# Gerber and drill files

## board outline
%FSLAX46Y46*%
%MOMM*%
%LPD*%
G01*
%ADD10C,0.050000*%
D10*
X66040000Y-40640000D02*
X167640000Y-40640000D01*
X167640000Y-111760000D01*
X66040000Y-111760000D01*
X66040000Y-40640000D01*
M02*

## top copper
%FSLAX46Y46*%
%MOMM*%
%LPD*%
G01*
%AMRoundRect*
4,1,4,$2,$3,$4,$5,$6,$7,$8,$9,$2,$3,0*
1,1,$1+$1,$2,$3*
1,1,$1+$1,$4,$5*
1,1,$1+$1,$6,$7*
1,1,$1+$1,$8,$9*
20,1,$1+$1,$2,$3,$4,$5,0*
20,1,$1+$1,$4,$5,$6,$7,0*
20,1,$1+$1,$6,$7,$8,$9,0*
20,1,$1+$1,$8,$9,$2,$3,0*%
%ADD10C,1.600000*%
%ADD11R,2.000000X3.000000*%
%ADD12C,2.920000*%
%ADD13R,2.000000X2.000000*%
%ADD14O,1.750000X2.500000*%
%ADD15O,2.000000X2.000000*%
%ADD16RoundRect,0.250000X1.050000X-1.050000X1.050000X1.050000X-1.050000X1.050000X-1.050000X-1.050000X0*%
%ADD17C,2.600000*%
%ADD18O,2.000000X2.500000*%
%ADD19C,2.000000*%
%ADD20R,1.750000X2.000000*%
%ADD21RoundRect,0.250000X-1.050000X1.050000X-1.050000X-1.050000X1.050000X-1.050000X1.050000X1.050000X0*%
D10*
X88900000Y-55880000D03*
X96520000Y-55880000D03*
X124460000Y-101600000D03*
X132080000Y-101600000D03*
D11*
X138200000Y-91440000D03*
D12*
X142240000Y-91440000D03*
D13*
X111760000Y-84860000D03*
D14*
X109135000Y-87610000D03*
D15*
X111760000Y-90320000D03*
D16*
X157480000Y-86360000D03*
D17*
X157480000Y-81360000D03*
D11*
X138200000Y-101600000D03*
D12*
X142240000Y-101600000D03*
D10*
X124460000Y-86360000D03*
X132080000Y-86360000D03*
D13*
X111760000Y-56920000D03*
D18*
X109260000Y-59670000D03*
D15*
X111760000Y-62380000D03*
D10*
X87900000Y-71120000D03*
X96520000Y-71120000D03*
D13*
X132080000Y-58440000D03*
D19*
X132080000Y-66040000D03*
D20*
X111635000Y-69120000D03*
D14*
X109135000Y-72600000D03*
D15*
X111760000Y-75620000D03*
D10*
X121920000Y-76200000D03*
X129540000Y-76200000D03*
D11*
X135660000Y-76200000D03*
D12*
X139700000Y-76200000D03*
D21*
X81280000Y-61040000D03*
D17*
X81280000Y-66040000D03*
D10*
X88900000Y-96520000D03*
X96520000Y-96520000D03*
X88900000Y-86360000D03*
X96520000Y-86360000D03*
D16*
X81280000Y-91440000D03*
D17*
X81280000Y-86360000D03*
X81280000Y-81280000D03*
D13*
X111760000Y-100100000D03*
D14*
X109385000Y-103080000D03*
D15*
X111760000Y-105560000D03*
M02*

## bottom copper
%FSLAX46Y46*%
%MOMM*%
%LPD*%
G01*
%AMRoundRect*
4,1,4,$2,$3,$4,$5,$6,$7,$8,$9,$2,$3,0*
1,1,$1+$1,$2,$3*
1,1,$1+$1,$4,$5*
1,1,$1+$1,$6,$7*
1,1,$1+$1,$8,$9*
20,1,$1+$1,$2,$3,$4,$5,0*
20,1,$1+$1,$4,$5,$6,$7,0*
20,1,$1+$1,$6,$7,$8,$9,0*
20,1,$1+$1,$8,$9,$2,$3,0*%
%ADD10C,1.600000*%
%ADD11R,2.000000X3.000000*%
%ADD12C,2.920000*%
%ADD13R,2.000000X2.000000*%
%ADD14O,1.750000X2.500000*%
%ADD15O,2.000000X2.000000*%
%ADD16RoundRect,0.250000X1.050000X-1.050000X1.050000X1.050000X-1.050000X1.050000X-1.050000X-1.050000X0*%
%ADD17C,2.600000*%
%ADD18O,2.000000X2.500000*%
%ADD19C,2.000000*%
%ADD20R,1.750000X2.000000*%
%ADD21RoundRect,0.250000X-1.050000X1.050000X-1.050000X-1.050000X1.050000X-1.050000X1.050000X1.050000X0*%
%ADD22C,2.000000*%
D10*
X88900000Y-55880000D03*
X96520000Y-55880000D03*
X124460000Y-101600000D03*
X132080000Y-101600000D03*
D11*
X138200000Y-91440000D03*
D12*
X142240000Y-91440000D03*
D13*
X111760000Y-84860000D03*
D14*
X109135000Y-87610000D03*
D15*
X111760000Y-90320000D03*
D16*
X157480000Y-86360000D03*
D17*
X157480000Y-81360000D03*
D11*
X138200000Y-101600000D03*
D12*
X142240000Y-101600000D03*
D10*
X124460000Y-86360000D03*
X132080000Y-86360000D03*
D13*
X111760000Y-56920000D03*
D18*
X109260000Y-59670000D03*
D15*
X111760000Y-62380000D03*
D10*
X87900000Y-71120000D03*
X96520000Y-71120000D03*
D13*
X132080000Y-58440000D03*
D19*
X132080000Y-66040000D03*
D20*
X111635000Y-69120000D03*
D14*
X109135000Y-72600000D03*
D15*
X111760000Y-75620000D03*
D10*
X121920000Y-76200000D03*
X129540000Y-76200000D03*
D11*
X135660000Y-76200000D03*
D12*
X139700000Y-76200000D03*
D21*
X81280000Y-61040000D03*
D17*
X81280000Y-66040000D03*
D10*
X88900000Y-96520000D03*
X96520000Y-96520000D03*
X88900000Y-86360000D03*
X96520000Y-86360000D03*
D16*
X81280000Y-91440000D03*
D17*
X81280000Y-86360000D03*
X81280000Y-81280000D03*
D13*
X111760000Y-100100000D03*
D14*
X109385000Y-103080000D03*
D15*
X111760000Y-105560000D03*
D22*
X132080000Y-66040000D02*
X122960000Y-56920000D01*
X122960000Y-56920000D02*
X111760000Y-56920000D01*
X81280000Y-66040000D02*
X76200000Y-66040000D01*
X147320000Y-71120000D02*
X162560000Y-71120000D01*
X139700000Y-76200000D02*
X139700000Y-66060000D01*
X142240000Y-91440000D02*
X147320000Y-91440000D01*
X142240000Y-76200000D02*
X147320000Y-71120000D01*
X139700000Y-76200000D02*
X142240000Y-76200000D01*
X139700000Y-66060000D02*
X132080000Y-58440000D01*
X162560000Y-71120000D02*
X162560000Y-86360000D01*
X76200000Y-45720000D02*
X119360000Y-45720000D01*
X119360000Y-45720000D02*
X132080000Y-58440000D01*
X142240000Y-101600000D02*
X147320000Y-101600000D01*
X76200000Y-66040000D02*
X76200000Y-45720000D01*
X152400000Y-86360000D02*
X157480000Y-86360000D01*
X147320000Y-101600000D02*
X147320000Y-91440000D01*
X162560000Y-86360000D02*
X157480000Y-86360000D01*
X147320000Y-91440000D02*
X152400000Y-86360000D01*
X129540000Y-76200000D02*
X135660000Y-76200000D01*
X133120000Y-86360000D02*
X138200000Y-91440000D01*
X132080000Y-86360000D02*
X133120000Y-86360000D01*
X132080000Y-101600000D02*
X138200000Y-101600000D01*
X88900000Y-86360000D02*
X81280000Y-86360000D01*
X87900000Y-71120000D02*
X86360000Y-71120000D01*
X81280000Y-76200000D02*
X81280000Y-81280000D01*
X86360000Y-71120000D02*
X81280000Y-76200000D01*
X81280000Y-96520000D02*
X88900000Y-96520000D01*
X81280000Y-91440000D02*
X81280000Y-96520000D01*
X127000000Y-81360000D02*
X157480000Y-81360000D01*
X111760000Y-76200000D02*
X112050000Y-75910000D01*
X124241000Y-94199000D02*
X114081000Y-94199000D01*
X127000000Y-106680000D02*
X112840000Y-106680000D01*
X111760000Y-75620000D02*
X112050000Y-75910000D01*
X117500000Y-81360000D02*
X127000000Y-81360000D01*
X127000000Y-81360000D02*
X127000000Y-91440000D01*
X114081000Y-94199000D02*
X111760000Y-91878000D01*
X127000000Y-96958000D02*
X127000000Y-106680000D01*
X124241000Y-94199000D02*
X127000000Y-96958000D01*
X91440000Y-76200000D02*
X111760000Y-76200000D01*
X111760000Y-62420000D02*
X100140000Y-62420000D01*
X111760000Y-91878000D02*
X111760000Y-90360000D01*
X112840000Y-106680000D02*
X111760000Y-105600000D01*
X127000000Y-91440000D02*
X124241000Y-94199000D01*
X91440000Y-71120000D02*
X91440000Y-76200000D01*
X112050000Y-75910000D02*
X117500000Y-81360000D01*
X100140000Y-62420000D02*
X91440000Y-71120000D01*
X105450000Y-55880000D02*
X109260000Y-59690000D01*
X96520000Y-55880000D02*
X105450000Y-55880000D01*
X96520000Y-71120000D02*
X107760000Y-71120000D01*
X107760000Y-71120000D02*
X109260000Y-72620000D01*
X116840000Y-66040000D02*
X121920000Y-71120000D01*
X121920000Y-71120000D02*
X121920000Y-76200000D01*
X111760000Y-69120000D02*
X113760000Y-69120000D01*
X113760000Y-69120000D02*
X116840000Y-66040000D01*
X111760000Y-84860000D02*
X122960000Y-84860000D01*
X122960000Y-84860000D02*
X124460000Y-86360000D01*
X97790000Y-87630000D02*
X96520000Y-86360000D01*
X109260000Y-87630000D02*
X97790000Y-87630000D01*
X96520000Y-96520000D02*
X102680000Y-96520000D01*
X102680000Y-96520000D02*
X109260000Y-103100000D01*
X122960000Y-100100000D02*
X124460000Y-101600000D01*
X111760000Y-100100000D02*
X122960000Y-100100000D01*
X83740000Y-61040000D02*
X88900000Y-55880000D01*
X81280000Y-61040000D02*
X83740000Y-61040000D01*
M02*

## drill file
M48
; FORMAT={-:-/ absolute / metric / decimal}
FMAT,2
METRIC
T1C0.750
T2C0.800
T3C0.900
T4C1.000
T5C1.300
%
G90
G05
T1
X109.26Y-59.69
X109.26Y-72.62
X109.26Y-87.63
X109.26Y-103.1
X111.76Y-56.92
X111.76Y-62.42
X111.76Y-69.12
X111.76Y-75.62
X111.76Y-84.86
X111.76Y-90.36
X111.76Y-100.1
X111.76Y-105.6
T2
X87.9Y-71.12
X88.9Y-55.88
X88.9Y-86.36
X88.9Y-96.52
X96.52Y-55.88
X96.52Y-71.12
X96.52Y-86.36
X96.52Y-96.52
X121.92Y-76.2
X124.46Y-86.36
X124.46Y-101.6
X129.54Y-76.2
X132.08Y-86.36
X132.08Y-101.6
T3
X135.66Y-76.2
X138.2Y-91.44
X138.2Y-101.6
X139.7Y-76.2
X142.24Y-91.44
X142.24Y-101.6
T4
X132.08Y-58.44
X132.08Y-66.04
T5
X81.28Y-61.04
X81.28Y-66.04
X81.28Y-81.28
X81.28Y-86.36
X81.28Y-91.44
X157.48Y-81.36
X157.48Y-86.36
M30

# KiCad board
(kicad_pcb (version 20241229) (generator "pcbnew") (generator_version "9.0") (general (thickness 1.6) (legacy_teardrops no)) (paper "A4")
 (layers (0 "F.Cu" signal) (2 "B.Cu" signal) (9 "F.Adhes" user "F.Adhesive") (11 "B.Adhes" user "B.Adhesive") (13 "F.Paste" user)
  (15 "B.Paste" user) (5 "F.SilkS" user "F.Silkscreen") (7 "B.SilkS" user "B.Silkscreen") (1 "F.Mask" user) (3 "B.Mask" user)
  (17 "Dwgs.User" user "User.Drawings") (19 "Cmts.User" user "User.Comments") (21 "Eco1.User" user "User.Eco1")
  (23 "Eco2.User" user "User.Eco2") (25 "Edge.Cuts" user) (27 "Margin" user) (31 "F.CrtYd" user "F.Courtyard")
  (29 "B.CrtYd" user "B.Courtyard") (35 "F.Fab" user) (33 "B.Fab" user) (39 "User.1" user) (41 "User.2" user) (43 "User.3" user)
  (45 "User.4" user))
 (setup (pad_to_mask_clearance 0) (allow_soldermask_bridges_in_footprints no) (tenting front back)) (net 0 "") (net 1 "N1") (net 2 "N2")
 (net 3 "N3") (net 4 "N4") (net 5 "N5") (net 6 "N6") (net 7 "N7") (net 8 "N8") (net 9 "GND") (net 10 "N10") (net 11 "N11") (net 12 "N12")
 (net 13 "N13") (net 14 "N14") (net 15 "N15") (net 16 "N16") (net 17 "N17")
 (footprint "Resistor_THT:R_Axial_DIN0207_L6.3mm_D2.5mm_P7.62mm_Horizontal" (layer "F.Cu") (at 88.9 55.88)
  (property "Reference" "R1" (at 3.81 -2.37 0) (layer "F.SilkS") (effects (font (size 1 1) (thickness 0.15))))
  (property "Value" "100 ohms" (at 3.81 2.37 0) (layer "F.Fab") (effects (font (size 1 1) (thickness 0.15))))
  (pad "1" thru_hole circle (at 0 0) (size 1.6 1.6) (drill 0.8) (layers "*.Cu" "*.Mask") (remove_unused_layers no) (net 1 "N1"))
  (pad "2" thru_hole circle (at 7.62 0) (size 1.6 1.6) (drill 0.8) (layers "*.Cu" "*.Mask") (remove_unused_layers no) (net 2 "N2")))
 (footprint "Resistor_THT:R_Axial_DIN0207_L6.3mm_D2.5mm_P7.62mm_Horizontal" (layer "F.Cu") (at 124.46 101.6)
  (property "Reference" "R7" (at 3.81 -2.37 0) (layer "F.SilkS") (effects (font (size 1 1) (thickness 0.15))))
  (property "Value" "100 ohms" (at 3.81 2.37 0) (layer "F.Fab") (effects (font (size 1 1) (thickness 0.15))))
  (pad "1" thru_hole circle (at 0 0) (size 1.6 1.6) (drill 0.8) (layers "*.Cu" "*.Mask") (remove_unused_layers no) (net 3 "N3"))
  (pad "2" thru_hole circle (at 7.62 0) (size 1.6 1.6) (drill 0.8) (layers "*.Cu" "*.Mask") (remove_unused_layers no) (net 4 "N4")))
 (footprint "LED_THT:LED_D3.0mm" (layer "F.Cu") (at 139.7 91.44)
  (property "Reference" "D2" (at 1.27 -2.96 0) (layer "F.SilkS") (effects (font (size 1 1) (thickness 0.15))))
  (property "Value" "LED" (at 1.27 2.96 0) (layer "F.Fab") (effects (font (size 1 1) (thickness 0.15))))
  (pad "1" thru_hole rect (at -1.5 0) (size 2 3) (drill 0.9) (layers "*.Cu" "*.Mask") (remove_unused_layers no) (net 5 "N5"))
  (pad "2" thru_hole circle (at 2.54 0) (size 2.92 2.92) (drill 0.9) (layers "*.Cu" "*.Mask") (remove_unused_layers no) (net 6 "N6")))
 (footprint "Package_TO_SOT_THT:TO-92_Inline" (layer "F.Cu") (at 111.76 86.36 -90)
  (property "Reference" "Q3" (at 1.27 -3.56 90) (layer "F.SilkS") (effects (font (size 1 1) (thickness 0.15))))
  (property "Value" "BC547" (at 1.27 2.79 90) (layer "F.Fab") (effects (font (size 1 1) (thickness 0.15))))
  (pad "1" thru_hole rect (at -1.5 0 270) (size 2 2) (drill 0.75) (layers "*.Cu" "*.Mask") (remove_unused_layers no) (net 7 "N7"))
  (pad "2" thru_hole oval (at 1.27 2.5 270) (size 2.5 1.75) (drill 0.75 (offset -0.02 0.125)) (layers "*.Cu" "*.Mask")
   (remove_unused_layers no) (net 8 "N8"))
  (pad "3" thru_hole oval (at 4 0 270) (size 2 2) (drill 0.75 (offset -0.04 0)) (layers "*.Cu" "*.Mask") (remove_unused_layers no)
   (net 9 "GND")))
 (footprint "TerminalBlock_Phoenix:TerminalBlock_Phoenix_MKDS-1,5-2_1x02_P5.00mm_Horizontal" (layer "F.Cu") (at 157.48 86.36 90)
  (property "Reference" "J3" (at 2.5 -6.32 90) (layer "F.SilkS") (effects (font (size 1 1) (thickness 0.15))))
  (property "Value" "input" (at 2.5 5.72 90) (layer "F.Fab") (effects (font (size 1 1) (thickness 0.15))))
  (pad "1" thru_hole roundrect (at 0 0 90) (size 2.6 2.6) (drill 1.3) (layers "*.Cu" "*.Mask") (remove_unused_layers no)
   (roundrect_rratio 0.096154) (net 6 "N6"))
  (pad "2" thru_hole circle (at 5 0 90) (size 2.6 2.6) (drill 1.3) (layers "*.Cu" "*.Mask") (remove_unused_layers no) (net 9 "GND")))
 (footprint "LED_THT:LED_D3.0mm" (layer "F.Cu") (at 139.7 101.6)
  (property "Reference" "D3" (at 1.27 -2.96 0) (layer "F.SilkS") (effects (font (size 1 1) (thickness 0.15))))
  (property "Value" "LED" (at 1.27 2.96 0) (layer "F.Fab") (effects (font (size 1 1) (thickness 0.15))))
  (pad "1" thru_hole rect (at -1.5 0) (size 2 3) (drill 0.9) (layers "*.Cu" "*.Mask") (remove_unused_layers no) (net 4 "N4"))
  (pad "2" thru_hole circle (at 2.54 0) (size 2.92 2.92) (drill 0.9) (layers "*.Cu" "*.Mask") (remove_unused_layers no) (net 6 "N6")))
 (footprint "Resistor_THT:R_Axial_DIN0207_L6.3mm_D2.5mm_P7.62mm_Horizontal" (layer "F.Cu") (at 124.46 86.36)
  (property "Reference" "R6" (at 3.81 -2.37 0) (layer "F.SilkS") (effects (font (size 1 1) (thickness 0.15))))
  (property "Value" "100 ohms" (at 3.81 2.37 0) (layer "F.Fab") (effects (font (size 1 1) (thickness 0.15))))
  (pad "1" thru_hole circle (at 0 0) (size 1.6 1.6) (drill 0.8) (layers "*.Cu" "*.Mask") (remove_unused_layers no) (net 7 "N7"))
  (pad "2" thru_hole circle (at 7.62 0) (size 1.6 1.6) (drill 0.8) (layers "*.Cu" "*.Mask") (remove_unused_layers no) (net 5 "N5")))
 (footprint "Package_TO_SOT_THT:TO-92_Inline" (layer "F.Cu") (at 111.76 58.42 -90)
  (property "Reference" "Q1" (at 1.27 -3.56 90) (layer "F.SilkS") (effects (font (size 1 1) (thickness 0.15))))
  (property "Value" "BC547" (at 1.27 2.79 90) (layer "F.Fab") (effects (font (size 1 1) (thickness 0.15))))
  (pad "1" thru_hole rect (at -1.5 0 270) (size 2 2) (drill 0.75) (layers "*.Cu" "*.Mask") (remove_unused_layers no) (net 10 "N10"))
  (pad "2" thru_hole oval (at 1.27 2.5 270) (size 2.5 2) (drill 0.75 (offset -0.02 0)) (layers "*.Cu" "*.Mask") (remove_unused_layers no)
   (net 2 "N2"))
  (pad "3" thru_hole oval (at 4 0 270) (size 2 2) (drill 0.75 (offset -0.04 0)) (layers "*.Cu" "*.Mask") (remove_unused_layers no)
   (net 9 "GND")))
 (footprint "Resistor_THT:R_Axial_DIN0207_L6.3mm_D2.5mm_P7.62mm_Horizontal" (layer "F.Cu") (at 88.9 71.12)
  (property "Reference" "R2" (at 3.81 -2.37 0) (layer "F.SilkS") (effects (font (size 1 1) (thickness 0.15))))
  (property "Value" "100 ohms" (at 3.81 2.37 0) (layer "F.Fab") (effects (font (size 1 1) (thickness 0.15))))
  (pad "1" thru_hole circle (at -1 0) (size 1.6 1.6) (drill 0.8) (layers "*.Cu" "*.Mask") (remove_unused_layers no) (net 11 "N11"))
  (pad "2" thru_hole circle (at 7.62 0) (size 1.6 1.6) (drill 0.8) (layers "*.Cu" "*.Mask") (remove_unused_layers no) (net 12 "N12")))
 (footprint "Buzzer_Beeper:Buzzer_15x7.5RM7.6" (layer "F.Cu") (at 132.08 58.44 -90)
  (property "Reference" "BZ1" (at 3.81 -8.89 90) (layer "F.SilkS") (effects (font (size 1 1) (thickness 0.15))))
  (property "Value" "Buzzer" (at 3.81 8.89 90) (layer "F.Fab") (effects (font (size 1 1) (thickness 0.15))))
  (pad "1" thru_hole rect (at 0 0 270) (size 2 2) (drill 1) (layers "*.Cu" "*.Mask") (remove_unused_layers no) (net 6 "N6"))
  (pad "2" thru_hole circle (at 7.6 0 270) (size 2 2) (drill 1) (layers "*.Cu" "*.Mask") (remove_unused_layers no) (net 10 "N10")))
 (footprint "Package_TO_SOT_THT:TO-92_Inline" (layer "F.Cu") (at 111.76 71.12 -90)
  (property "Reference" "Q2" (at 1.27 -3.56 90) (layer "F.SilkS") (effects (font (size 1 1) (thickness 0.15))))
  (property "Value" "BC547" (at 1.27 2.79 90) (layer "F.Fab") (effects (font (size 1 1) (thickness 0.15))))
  (pad "1" thru_hole rect (at -2 0 270) (size 2 1.75) (drill 0.75 (offset 0 0.125)) (layers "*.Cu" "*.Mask") (remove_unused_layers no)
   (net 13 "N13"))
  (pad "2" thru_hole oval (at 1.5 2.5 270) (size 2.5 1.75) (drill 0.75 (offset -0.02 0.125)) (layers "*.Cu" "*.Mask")
   (remove_unused_layers no) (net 12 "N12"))
  (pad "3" thru_hole oval (at 4.5 0 270) (size 2 2) (drill 0.75) (layers "*.Cu" "*.Mask") (remove_unused_layers no) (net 9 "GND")))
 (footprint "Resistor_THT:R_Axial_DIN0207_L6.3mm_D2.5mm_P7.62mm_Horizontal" (layer "F.Cu") (at 121.92 76.2)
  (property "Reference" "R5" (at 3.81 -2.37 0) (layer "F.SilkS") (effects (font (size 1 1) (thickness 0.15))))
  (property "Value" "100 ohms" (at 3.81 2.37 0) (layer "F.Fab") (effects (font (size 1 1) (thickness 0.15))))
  (pad "1" thru_hole circle (at 0 0) (size 1.6 1.6) (drill 0.8) (layers "*.Cu" "*.Mask") (remove_unused_layers no) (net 13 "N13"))
  (pad "2" thru_hole circle (at 7.62 0) (size 1.6 1.6) (drill 0.8) (layers "*.Cu" "*.Mask") (remove_unused_layers no) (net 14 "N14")))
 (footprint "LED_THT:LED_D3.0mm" (layer "F.Cu") (at 137.16 76.2)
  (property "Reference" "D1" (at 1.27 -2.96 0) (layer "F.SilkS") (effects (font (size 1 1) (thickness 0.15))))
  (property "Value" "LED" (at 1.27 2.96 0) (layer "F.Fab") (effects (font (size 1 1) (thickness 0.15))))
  (pad "1" thru_hole rect (at -1.5 0) (size 2 3) (drill 0.9) (layers "*.Cu" "*.Mask") (remove_unused_layers no) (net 14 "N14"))
  (pad "2" thru_hole circle (at 2.54 0) (size 2.92 2.92) (drill 0.9) (layers "*.Cu" "*.Mask") (remove_unused_layers no) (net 6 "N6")))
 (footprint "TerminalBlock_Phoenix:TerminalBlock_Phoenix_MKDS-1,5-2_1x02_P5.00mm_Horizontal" (layer "F.Cu") (at 81.28 61.04 -90)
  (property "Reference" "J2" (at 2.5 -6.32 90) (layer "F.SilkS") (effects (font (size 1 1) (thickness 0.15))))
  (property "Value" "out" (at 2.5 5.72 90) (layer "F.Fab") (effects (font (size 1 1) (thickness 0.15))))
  (pad "1" thru_hole roundrect (at 0 0 270) (size 2.6 2.6) (drill 1.3) (layers "*.Cu" "*.Mask") (remove_unused_layers no)
   (roundrect_rratio 0.096154) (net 1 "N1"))
  (pad "2" thru_hole circle (at 5 0 270) (size 2.6 2.6) (drill 1.3) (layers "*.Cu" "*.Mask") (remove_unused_layers no) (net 6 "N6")))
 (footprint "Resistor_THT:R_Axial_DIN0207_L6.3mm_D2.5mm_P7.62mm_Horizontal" (layer "F.Cu") (at 88.9 96.52)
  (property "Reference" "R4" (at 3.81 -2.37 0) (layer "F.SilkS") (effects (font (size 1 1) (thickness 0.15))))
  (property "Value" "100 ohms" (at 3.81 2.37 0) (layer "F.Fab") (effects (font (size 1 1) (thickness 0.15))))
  (pad "1" thru_hole circle (at 0 0) (size 1.6 1.6) (drill 0.8) (layers "*.Cu" "*.Mask") (remove_unused_layers no) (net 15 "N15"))
  (pad "2" thru_hole circle (at 7.62 0) (size 1.6 1.6) (drill 0.8) (layers "*.Cu" "*.Mask") (remove_unused_layers no) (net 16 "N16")))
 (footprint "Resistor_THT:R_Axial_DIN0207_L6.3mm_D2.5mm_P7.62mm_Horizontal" (layer "F.Cu") (at 88.9 86.36)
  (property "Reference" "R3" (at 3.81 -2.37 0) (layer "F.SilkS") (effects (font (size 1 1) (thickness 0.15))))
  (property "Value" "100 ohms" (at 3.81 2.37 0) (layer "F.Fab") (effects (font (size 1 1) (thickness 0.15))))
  (pad "1" thru_hole circle (at 0 0) (size 1.6 1.6) (drill 0.8) (layers "*.Cu" "*.Mask") (remove_unused_layers no) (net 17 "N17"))
  (pad "2" thru_hole circle (at 7.62 0) (size 1.6 1.6) (drill 0.8) (layers "*.Cu" "*.Mask") (remove_unused_layers no) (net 8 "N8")))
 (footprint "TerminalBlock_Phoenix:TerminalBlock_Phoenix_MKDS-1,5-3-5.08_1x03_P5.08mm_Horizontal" (layer "F.Cu") (at 81.28 91.44 90)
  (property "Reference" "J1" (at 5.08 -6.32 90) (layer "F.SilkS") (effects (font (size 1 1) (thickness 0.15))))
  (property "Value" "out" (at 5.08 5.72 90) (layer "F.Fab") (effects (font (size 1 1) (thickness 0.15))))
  (pad "1" thru_hole roundrect (at 0 0 90) (size 2.6 2.6) (drill 1.3) (layers "*.Cu" "*.Mask") (remove_unused_layers no)
   (roundrect_rratio 0.096154) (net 15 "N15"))
  (pad "2" thru_hole circle (at 5.08 0 90) (size 2.6 2.6) (drill 1.3) (layers "*.Cu" "*.Mask") (remove_unused_layers no) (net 17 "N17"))
  (pad "3" thru_hole circle (at 10.16 0 90) (size 2.6 2.6) (drill 1.3) (layers "*.Cu" "*.Mask") (remove_unused_layers no) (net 11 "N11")))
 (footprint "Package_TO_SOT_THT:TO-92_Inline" (layer "F.Cu") (at 111.76 101.6 -90)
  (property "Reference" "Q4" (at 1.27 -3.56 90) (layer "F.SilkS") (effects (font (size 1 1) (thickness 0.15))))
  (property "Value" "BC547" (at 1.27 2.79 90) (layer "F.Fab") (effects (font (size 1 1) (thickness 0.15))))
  (pad "1" thru_hole rect (at -1.5 0 270) (size 2 2) (drill 0.75) (layers "*.Cu" "*.Mask") (remove_unused_layers no) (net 3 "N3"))
  (pad "2" thru_hole oval (at 1.5 2.5 270) (size 2.5 1.75) (drill 0.75 (offset -0.02 -0.125)) (layers "*.Cu" "*.Mask")
   (remove_unused_layers no) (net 16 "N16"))
  (pad "3" thru_hole oval (at 4 0 270) (size 2 2) (drill 0.75 (offset -0.04 0)) (layers "*.Cu" "*.Mask") (remove_unused_layers no)
   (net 9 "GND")))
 (gr_rect (start 66.04 40.64) (end 167.64 111.76) (stroke (width 0.05) (type default)) (fill no) (layer "Edge.Cuts"))
 (segment (start 132.08 66.04) (end 122.96 56.92) (width 2) (layer "B.Cu") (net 10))
 (segment (start 122.96 56.92) (end 111.76 56.92) (width 2) (layer "B.Cu") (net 10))
 (segment (start 81.28 66.04) (end 76.2 66.04) (width 2) (layer "B.Cu") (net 6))
 (segment (start 147.32 71.12) (end 162.56 71.12) (width 2) (layer "B.Cu") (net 6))
 (segment (start 139.7 76.2) (end 139.7 66.06) (width 2) (layer "B.Cu") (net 6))
 (segment (start 142.24 91.44) (end 147.32 91.44) (width 2) (layer "B.Cu") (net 6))
 (segment (start 142.24 76.2) (end 147.32 71.12) (width 2) (layer "B.Cu") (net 6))
 (segment (start 139.7 76.2) (end 142.24 76.2) (width 2) (layer "B.Cu") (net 6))
 (segment (start 139.7 66.06) (end 132.08 58.44) (width 2) (layer "B.Cu") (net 6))
 (segment (start 162.56 71.12) (end 162.56 86.36) (width 2) (layer "B.Cu") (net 6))
 (segment (start 76.2 45.72) (end 119.36 45.72) (width 2) (layer "B.Cu") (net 6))
 (segment (start 119.36 45.72) (end 132.08 58.44) (width 2) (layer "B.Cu") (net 6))
 (segment (start 142.24 101.6) (end 147.32 101.6) (width 2) (layer "B.Cu") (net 6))
 (segment (start 76.2 66.04) (end 76.2 45.72) (width 2) (layer "B.Cu") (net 6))
 (segment (start 152.4 86.36) (end 157.48 86.36) (width 2) (layer "B.Cu") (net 6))
 (segment (start 147.32 101.6) (end 147.32 91.44) (width 2) (layer "B.Cu") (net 6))
 (segment (start 162.56 86.36) (end 157.48 86.36) (width 2) (layer "B.Cu") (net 6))
 (segment (start 147.32 91.44) (end 152.4 86.36) (width 2) (layer "B.Cu") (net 6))
 (segment (start 129.54 76.2) (end 135.66 76.2) (width 2) (layer "B.Cu") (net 14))
 (segment (start 133.12 86.36) (end 138.2 91.44) (width 2) (layer "B.Cu") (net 5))
 (segment (start 132.08 86.36) (end 133.12 86.36) (width 2) (layer "B.Cu") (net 5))
 (segment (start 132.08 101.6) (end 138.2 101.6) (width 2) (layer "B.Cu") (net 4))
 (segment (start 88.9 86.36) (end 81.28 86.36) (width 2) (layer "B.Cu") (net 17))
 (segment (start 87.9 71.12) (end 86.36 71.12) (width 2) (layer "B.Cu") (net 11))
 (segment (start 81.28 76.2) (end 81.28 81.28) (width 2) (layer "B.Cu") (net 11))
 (segment (start 86.36 71.12) (end 81.28 76.2) (width 2) (layer "B.Cu") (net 11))
 (segment (start 81.28 96.52) (end 88.9 96.52) (width 2) (layer "B.Cu") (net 15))
 (segment (start 81.28 91.44) (end 81.28 96.52) (width 2) (layer "B.Cu") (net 15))
 (segment (start 127 81.36) (end 157.48 81.36) (width 2) (layer "B.Cu") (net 9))
 (segment (start 111.76 76.2) (end 112.05 75.91) (width 2) (layer "B.Cu") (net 9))
 (segment (start 124.241 94.199) (end 114.081 94.199) (width 2) (layer "B.Cu") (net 9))
 (segment (start 127 106.68) (end 112.84 106.68) (width 2) (layer "B.Cu") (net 9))
 (segment (start 111.76 75.62) (end 112.05 75.91) (width 2) (layer "B.Cu") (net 9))
 (segment (start 117.5 81.36) (end 127 81.36) (width 2) (layer "B.Cu") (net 9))
 (segment (start 127 81.36) (end 127 91.44) (width 2) (layer "B.Cu") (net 9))
 (segment (start 114.081 94.199) (end 111.76 91.878) (width 2) (layer "B.Cu") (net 9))
 (segment (start 127 96.958) (end 127 106.68) (width 2) (layer "B.Cu") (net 9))
 (segment (start 124.241 94.199) (end 127 96.958) (width 2) (layer "B.Cu") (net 9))
 (segment (start 91.44 76.2) (end 111.76 76.2) (width 2) (layer "B.Cu") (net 9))
 (segment (start 111.76 62.42) (end 100.14 62.42) (width 2) (layer "B.Cu") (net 9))
 (segment (start 111.76 91.878) (end 111.76 90.36) (width 2) (layer "B.Cu") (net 9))
 (segment (start 112.84 106.68) (end 111.76 105.6) (width 2) (layer "B.Cu") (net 9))
 (segment (start 127 91.44) (end 124.241 94.199) (width 2) (layer "B.Cu") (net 9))
 (segment (start 91.44 71.12) (end 91.44 76.2) (width 2) (layer "B.Cu") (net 9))
 (segment (start 112.05 75.91) (end 117.5 81.36) (width 2) (layer "B.Cu") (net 9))
 (segment (start 100.14 62.42) (end 91.44 71.12) (width 2) (layer "B.Cu") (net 9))
 (segment (start 105.45 55.88) (end 109.26 59.69) (width 2) (layer "B.Cu") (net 2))
 (segment (start 96.52 55.88) (end 105.45 55.88) (width 2) (layer "B.Cu") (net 2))
 (segment (start 96.52 71.12) (end 107.76 71.12) (width 2) (layer "B.Cu") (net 12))
 (segment (start 107.76 71.12) (end 109.26 72.62) (width 2) (layer "B.Cu") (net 12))
 (segment (start 116.84 66.04) (end 121.92 71.12) (width 2) (layer "B.Cu") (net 13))
 (segment (start 121.92 71.12) (end 121.92 76.2) (width 2) (layer "B.Cu") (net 13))
 (segment (start 111.76 69.12) (end 113.76 69.12) (width 2) (layer "B.Cu") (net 13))
 (segment (start 113.76 69.12) (end 116.84 66.04) (width 2) (layer "B.Cu") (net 13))
 (segment (start 111.76 84.86) (end 122.96 84.86) (width 2) (layer "B.Cu") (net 7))
 (segment (start 122.96 84.86) (end 124.46 86.36) (width 2) (layer "B.Cu") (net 7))
 (segment (start 97.79 87.63) (end 96.52 86.36) (width 2) (layer "B.Cu") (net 8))
 (segment (start 109.26 87.63) (end 97.79 87.63) (width 2) (layer "B.Cu") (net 8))
 (segment (start 96.52 96.52) (end 102.68 96.52) (width 2) (layer "B.Cu") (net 16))
 (segment (start 102.68 96.52) (end 109.26 103.1) (width 2) (layer "B.Cu") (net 16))
 (segment (start 122.96 100.1) (end 124.46 101.6) (width 2) (layer "B.Cu") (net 3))
 (segment (start 111.76 100.1) (end 122.96 100.1) (width 2) (layer "B.Cu") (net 3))
 (segment (start 83.74 61.04) (end 88.9 55.88) (width 2) (layer "B.Cu") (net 1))
 (segment (start 81.28 61.04) (end 83.74 61.04) (width 2) (layer "B.Cu") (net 1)))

